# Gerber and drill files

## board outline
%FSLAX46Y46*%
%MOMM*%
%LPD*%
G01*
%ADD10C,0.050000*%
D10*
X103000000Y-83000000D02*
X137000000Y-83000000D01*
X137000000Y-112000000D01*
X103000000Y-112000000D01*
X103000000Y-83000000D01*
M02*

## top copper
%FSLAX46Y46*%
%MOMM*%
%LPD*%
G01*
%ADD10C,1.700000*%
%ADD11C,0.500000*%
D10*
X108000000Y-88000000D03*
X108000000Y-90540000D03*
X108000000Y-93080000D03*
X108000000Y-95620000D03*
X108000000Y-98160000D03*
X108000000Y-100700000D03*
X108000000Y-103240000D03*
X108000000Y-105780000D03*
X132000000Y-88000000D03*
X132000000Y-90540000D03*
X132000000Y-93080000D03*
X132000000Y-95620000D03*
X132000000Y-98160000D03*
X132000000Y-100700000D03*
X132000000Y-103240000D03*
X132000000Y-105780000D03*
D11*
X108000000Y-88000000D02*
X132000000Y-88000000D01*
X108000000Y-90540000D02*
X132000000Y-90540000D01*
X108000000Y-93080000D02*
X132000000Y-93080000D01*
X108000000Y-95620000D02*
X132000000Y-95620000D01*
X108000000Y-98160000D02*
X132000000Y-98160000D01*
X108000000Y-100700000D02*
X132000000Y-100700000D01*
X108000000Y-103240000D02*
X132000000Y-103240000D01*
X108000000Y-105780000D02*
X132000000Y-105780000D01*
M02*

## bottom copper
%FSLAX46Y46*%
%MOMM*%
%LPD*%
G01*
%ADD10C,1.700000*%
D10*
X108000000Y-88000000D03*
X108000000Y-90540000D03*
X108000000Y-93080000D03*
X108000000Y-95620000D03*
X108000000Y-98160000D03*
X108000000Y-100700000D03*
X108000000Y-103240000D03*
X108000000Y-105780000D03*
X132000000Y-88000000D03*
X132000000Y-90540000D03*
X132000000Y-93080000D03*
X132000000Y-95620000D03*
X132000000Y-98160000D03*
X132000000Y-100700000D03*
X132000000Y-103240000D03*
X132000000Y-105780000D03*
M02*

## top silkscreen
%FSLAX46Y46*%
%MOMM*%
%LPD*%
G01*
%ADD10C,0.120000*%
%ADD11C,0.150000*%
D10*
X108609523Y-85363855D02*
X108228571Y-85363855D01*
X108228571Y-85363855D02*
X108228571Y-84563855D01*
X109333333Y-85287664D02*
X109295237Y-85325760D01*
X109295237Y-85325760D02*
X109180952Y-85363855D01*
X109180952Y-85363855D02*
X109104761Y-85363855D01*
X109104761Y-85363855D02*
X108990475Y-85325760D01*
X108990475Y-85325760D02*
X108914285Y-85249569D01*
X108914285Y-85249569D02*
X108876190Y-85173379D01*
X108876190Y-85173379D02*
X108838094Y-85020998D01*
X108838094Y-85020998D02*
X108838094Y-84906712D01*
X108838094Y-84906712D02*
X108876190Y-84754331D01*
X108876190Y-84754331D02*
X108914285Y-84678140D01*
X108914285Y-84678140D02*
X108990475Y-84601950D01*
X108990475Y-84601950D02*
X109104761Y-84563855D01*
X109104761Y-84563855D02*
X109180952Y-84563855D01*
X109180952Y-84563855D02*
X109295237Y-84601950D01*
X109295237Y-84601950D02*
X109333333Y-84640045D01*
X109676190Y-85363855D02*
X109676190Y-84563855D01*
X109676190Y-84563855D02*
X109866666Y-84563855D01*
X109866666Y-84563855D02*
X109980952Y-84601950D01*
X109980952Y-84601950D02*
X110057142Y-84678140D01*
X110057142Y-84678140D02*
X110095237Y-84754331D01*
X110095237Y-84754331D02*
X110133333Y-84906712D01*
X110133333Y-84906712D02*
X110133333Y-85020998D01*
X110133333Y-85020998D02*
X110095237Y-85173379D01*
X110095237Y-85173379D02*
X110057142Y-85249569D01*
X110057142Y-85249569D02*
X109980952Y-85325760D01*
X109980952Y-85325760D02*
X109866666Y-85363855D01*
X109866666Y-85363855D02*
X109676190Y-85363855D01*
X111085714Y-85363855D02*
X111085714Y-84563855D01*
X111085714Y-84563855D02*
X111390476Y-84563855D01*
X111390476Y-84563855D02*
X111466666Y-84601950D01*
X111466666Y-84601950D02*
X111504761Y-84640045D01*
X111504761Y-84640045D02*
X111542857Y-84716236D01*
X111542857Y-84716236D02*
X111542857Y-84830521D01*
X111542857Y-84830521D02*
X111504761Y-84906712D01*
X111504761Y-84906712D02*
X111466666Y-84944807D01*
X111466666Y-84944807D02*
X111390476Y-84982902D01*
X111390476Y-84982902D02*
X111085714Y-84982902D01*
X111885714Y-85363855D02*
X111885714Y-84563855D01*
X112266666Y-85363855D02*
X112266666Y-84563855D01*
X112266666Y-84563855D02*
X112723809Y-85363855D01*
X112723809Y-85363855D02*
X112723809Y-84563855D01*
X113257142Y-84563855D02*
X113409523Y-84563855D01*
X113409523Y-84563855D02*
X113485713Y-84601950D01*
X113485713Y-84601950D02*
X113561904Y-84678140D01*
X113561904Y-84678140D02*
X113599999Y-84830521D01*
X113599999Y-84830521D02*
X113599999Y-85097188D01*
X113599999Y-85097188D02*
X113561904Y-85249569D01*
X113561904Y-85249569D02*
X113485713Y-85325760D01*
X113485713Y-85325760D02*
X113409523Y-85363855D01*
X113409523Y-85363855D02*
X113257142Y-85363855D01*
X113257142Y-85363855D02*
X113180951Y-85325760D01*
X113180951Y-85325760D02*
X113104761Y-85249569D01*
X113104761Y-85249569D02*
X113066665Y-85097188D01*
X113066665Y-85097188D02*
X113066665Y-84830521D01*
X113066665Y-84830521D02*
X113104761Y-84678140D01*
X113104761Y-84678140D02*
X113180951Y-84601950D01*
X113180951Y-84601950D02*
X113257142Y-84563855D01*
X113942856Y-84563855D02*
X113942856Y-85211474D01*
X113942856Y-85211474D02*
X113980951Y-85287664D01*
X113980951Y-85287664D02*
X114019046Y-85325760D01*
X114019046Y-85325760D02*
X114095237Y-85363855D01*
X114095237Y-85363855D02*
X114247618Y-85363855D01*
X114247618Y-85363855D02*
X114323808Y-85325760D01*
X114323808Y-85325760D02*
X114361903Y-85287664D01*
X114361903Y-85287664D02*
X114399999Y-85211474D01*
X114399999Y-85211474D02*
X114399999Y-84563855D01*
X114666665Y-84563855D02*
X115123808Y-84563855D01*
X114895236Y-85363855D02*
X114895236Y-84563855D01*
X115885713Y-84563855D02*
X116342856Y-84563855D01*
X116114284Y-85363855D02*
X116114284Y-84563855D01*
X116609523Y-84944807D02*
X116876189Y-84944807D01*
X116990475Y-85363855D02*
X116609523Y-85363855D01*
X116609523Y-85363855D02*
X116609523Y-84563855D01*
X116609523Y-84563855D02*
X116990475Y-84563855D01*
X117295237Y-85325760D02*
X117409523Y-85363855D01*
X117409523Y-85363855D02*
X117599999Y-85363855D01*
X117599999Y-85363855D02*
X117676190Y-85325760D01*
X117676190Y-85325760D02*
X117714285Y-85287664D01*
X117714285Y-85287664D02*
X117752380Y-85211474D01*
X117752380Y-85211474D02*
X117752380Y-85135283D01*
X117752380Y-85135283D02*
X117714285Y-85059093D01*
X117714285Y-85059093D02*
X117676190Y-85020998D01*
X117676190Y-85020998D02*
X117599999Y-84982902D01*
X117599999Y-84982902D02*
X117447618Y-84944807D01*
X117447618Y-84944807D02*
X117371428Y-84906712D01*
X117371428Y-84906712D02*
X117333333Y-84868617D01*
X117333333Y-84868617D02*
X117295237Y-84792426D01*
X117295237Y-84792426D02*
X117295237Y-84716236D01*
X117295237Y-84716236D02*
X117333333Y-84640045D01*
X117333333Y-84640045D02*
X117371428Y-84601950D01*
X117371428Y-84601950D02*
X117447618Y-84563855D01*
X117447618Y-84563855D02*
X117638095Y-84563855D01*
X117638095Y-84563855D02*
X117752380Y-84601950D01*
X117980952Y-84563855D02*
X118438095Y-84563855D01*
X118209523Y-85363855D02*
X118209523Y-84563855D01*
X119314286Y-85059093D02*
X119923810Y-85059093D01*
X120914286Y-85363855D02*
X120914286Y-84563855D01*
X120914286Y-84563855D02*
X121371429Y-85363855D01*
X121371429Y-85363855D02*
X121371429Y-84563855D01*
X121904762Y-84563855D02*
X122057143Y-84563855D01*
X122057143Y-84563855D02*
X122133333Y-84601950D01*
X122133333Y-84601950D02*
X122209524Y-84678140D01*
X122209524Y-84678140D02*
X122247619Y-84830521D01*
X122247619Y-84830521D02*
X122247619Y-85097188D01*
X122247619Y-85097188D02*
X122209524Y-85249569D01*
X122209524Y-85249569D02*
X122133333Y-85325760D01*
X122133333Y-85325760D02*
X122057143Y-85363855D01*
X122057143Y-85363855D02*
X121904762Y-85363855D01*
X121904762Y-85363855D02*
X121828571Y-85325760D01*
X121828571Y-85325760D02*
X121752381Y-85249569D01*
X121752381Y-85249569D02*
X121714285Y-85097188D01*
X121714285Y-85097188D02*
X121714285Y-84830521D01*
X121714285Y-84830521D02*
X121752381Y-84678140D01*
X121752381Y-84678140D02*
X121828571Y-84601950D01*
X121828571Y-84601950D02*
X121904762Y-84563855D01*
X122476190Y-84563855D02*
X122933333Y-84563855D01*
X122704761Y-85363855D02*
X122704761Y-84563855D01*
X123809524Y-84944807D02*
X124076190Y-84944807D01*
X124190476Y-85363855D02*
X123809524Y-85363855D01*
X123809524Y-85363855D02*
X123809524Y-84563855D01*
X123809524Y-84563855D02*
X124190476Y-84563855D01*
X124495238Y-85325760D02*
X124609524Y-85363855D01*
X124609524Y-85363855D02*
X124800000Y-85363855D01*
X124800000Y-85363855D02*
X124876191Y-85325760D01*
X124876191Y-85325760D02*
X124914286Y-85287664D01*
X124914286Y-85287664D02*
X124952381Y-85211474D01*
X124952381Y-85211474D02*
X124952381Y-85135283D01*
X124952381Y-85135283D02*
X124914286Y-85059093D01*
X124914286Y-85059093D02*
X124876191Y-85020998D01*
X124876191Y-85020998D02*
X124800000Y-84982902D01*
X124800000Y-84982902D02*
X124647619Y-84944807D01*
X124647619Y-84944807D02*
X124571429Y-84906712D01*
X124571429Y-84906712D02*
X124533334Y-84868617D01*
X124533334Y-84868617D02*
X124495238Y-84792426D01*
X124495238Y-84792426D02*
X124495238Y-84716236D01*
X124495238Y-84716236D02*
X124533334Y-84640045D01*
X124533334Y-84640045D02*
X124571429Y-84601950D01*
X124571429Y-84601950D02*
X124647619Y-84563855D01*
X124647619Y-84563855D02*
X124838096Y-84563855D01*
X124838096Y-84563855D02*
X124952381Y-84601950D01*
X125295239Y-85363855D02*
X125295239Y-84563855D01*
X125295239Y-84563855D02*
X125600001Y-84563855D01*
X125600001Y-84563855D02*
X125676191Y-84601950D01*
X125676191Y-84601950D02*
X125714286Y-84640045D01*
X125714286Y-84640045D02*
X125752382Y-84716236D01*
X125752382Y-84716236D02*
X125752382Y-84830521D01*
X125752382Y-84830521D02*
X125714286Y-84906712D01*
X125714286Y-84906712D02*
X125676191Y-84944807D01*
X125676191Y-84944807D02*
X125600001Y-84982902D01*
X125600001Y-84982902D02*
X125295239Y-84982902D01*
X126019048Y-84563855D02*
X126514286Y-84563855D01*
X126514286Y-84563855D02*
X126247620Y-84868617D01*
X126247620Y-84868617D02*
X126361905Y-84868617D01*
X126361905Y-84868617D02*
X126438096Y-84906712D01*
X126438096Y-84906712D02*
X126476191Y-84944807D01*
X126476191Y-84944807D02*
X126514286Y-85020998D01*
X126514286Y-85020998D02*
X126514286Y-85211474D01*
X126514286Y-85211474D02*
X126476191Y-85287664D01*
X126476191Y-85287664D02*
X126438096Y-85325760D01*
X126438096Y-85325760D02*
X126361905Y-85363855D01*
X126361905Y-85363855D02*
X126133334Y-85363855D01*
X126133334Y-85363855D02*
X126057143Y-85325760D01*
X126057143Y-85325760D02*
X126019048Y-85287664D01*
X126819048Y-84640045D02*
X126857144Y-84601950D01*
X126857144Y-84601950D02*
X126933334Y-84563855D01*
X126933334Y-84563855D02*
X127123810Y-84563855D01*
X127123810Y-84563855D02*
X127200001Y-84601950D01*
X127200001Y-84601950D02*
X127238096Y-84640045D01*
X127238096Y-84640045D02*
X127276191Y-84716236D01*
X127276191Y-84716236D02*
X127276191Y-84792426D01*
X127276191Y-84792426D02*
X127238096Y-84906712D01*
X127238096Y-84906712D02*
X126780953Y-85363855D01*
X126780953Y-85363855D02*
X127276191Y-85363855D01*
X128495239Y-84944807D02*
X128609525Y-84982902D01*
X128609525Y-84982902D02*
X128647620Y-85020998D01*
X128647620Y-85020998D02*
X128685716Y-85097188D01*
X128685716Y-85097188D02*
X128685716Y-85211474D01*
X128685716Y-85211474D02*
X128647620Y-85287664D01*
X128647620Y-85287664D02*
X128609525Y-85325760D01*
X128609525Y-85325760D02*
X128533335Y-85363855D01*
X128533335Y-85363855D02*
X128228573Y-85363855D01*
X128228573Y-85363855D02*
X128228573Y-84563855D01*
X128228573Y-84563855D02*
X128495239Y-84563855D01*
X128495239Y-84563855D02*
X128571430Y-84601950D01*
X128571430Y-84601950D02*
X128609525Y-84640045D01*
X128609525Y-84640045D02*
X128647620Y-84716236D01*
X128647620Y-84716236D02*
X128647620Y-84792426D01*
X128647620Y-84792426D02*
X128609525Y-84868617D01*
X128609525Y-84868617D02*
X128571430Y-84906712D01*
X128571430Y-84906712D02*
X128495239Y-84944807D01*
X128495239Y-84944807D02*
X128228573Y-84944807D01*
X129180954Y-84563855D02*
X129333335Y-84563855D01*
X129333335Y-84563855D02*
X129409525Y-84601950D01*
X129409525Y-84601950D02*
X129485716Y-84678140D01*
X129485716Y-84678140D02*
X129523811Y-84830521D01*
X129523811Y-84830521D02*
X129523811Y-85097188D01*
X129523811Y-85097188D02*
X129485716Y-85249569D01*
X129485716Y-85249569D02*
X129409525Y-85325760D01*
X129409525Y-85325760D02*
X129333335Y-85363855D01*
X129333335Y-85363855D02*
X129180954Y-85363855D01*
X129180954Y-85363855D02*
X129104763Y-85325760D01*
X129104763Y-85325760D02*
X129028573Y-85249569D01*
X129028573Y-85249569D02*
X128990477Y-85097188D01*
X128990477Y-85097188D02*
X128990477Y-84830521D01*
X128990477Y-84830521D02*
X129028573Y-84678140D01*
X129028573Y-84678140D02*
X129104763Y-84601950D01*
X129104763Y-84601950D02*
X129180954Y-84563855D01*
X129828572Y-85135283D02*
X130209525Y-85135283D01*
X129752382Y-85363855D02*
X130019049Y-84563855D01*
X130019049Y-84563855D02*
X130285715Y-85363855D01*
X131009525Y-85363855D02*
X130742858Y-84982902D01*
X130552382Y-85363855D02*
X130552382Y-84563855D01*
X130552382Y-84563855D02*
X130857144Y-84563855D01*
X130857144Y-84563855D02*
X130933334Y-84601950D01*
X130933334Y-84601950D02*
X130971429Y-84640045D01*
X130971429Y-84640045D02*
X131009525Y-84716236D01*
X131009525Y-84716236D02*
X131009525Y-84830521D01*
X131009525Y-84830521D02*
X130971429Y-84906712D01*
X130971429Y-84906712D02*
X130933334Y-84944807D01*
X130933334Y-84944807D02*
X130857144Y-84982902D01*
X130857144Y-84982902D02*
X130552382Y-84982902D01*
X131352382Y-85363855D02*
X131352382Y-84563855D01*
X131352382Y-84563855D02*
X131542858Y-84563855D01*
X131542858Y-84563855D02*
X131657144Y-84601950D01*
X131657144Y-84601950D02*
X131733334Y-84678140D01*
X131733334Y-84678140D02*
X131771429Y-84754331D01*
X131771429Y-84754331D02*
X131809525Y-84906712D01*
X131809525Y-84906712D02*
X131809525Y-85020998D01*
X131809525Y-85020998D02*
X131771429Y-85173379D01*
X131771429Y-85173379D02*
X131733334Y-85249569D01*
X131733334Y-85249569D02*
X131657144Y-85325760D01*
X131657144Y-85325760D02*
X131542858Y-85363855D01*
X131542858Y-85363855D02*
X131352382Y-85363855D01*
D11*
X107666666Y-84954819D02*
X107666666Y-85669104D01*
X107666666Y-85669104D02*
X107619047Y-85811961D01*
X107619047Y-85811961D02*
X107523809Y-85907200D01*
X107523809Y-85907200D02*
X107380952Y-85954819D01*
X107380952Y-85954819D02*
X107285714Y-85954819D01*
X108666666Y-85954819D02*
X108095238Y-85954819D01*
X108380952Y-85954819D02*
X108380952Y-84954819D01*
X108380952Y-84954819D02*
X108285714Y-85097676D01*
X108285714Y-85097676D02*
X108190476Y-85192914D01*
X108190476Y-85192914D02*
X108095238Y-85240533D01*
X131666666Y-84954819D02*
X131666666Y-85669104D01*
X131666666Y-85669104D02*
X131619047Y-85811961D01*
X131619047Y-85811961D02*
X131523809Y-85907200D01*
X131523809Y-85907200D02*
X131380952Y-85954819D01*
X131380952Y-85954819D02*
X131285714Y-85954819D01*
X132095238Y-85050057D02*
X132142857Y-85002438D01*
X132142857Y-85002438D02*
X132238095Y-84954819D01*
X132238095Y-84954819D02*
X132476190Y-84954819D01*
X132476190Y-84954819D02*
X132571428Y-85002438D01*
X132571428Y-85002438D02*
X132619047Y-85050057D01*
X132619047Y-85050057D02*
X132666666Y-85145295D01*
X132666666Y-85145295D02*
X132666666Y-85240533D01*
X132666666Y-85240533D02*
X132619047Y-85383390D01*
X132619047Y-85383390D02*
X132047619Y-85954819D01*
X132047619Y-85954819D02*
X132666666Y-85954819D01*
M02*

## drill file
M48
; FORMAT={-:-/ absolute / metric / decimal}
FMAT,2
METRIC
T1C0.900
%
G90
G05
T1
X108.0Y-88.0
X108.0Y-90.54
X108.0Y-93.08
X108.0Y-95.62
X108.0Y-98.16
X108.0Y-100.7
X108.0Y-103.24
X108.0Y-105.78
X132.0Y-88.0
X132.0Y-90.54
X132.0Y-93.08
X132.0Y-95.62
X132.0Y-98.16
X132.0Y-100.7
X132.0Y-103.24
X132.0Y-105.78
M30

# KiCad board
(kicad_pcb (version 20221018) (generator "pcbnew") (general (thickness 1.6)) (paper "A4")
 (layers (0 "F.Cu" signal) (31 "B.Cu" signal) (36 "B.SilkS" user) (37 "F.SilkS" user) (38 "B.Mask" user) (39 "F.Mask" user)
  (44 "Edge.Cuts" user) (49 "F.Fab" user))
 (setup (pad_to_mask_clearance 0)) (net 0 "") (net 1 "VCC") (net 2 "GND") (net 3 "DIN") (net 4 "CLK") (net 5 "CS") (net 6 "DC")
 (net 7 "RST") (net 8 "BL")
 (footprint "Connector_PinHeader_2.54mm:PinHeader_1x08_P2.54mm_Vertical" (layer "F.Cu") (at 108 88)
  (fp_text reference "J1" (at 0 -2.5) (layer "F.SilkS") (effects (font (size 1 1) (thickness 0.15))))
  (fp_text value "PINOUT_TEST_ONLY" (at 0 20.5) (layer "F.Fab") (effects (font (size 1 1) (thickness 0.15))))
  (pad "1" thru_hole circle (at 0 0) (size 1.7 1.7) (drill 0.9) (layers "*.Cu" "*.Mask") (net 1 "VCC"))
  (pad "2" thru_hole circle (at 0 2.54) (size 1.7 1.7) (drill 0.9) (layers "*.Cu" "*.Mask") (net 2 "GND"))
  (pad "3" thru_hole circle (at 0 5.08) (size 1.7 1.7) (drill 0.9) (layers "*.Cu" "*.Mask") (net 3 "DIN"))
  (pad "4" thru_hole circle (at 0 7.62) (size 1.7 1.7) (drill 0.9) (layers "*.Cu" "*.Mask") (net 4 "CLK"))
  (pad "5" thru_hole circle (at 0 10.16) (size 1.7 1.7) (drill 0.9) (layers "*.Cu" "*.Mask") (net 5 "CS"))
  (pad "6" thru_hole circle (at 0 12.7) (size 1.7 1.7) (drill 0.9) (layers "*.Cu" "*.Mask") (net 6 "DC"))
  (pad "7" thru_hole circle (at 0 15.24) (size 1.7 1.7) (drill 0.9) (layers "*.Cu" "*.Mask") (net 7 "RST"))
  (pad "8" thru_hole circle (at 0 17.78) (size 1.7 1.7) (drill 0.9) (layers "*.Cu" "*.Mask") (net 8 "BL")))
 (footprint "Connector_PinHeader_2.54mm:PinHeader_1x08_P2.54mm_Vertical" (layer "F.Cu") (at 132 88)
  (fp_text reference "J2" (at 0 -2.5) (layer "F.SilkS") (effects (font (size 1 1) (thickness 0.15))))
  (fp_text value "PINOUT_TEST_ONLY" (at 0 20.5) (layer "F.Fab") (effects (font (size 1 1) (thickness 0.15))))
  (pad "1" thru_hole circle (at 0 0) (size 1.7 1.7) (drill 0.9) (layers "*.Cu" "*.Mask") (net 1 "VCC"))
  (pad "2" thru_hole circle (at 0 2.54) (size 1.7 1.7) (drill 0.9) (layers "*.Cu" "*.Mask") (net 2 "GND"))
  (pad "3" thru_hole circle (at 0 5.08) (size 1.7 1.7) (drill 0.9) (layers "*.Cu" "*.Mask") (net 3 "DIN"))
  (pad "4" thru_hole circle (at 0 7.62) (size 1.7 1.7) (drill 0.9) (layers "*.Cu" "*.Mask") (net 4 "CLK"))
  (pad "5" thru_hole circle (at 0 10.16) (size 1.7 1.7) (drill 0.9) (layers "*.Cu" "*.Mask") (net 5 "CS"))
  (pad "6" thru_hole circle (at 0 12.7) (size 1.7 1.7) (drill 0.9) (layers "*.Cu" "*.Mask") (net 6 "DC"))
  (pad "7" thru_hole circle (at 0 15.24) (size 1.7 1.7) (drill 0.9) (layers "*.Cu" "*.Mask") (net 7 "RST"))
  (pad "8" thru_hole circle (at 0 17.78) (size 1.7 1.7) (drill 0.9) (layers "*.Cu" "*.Mask") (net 8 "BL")))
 (segment (start 108 88) (end 132 88) (width 0.5) (layer "F.Cu") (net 1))
 (segment (start 108 90.54) (end 132 90.54) (width 0.5) (layer "F.Cu") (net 2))
 (segment (start 108 93.08) (end 132 93.08) (width 0.5) (layer "F.Cu") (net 3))
 (segment (start 108 95.62) (end 132 95.62) (width 0.5) (layer "F.Cu") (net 4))
 (segment (start 108 98.16) (end 132 98.16) (width 0.5) (layer "F.Cu") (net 5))
 (segment (start 108 100.7) (end 132 100.7) (width 0.5) (layer "F.Cu") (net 6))
 (segment (start 108 103.24) (end 132 103.24) (width 0.5) (layer "F.Cu") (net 7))
 (segment (start 108 105.78) (end 132 105.78) (width 0.5) (layer "F.Cu") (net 8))
 (gr_rect (start 103 83) (end 137 112) (stroke (width 0.05) (type default)) (fill none) (layer "Edge.Cuts"))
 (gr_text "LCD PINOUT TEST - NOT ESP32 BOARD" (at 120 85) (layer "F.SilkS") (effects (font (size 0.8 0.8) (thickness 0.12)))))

